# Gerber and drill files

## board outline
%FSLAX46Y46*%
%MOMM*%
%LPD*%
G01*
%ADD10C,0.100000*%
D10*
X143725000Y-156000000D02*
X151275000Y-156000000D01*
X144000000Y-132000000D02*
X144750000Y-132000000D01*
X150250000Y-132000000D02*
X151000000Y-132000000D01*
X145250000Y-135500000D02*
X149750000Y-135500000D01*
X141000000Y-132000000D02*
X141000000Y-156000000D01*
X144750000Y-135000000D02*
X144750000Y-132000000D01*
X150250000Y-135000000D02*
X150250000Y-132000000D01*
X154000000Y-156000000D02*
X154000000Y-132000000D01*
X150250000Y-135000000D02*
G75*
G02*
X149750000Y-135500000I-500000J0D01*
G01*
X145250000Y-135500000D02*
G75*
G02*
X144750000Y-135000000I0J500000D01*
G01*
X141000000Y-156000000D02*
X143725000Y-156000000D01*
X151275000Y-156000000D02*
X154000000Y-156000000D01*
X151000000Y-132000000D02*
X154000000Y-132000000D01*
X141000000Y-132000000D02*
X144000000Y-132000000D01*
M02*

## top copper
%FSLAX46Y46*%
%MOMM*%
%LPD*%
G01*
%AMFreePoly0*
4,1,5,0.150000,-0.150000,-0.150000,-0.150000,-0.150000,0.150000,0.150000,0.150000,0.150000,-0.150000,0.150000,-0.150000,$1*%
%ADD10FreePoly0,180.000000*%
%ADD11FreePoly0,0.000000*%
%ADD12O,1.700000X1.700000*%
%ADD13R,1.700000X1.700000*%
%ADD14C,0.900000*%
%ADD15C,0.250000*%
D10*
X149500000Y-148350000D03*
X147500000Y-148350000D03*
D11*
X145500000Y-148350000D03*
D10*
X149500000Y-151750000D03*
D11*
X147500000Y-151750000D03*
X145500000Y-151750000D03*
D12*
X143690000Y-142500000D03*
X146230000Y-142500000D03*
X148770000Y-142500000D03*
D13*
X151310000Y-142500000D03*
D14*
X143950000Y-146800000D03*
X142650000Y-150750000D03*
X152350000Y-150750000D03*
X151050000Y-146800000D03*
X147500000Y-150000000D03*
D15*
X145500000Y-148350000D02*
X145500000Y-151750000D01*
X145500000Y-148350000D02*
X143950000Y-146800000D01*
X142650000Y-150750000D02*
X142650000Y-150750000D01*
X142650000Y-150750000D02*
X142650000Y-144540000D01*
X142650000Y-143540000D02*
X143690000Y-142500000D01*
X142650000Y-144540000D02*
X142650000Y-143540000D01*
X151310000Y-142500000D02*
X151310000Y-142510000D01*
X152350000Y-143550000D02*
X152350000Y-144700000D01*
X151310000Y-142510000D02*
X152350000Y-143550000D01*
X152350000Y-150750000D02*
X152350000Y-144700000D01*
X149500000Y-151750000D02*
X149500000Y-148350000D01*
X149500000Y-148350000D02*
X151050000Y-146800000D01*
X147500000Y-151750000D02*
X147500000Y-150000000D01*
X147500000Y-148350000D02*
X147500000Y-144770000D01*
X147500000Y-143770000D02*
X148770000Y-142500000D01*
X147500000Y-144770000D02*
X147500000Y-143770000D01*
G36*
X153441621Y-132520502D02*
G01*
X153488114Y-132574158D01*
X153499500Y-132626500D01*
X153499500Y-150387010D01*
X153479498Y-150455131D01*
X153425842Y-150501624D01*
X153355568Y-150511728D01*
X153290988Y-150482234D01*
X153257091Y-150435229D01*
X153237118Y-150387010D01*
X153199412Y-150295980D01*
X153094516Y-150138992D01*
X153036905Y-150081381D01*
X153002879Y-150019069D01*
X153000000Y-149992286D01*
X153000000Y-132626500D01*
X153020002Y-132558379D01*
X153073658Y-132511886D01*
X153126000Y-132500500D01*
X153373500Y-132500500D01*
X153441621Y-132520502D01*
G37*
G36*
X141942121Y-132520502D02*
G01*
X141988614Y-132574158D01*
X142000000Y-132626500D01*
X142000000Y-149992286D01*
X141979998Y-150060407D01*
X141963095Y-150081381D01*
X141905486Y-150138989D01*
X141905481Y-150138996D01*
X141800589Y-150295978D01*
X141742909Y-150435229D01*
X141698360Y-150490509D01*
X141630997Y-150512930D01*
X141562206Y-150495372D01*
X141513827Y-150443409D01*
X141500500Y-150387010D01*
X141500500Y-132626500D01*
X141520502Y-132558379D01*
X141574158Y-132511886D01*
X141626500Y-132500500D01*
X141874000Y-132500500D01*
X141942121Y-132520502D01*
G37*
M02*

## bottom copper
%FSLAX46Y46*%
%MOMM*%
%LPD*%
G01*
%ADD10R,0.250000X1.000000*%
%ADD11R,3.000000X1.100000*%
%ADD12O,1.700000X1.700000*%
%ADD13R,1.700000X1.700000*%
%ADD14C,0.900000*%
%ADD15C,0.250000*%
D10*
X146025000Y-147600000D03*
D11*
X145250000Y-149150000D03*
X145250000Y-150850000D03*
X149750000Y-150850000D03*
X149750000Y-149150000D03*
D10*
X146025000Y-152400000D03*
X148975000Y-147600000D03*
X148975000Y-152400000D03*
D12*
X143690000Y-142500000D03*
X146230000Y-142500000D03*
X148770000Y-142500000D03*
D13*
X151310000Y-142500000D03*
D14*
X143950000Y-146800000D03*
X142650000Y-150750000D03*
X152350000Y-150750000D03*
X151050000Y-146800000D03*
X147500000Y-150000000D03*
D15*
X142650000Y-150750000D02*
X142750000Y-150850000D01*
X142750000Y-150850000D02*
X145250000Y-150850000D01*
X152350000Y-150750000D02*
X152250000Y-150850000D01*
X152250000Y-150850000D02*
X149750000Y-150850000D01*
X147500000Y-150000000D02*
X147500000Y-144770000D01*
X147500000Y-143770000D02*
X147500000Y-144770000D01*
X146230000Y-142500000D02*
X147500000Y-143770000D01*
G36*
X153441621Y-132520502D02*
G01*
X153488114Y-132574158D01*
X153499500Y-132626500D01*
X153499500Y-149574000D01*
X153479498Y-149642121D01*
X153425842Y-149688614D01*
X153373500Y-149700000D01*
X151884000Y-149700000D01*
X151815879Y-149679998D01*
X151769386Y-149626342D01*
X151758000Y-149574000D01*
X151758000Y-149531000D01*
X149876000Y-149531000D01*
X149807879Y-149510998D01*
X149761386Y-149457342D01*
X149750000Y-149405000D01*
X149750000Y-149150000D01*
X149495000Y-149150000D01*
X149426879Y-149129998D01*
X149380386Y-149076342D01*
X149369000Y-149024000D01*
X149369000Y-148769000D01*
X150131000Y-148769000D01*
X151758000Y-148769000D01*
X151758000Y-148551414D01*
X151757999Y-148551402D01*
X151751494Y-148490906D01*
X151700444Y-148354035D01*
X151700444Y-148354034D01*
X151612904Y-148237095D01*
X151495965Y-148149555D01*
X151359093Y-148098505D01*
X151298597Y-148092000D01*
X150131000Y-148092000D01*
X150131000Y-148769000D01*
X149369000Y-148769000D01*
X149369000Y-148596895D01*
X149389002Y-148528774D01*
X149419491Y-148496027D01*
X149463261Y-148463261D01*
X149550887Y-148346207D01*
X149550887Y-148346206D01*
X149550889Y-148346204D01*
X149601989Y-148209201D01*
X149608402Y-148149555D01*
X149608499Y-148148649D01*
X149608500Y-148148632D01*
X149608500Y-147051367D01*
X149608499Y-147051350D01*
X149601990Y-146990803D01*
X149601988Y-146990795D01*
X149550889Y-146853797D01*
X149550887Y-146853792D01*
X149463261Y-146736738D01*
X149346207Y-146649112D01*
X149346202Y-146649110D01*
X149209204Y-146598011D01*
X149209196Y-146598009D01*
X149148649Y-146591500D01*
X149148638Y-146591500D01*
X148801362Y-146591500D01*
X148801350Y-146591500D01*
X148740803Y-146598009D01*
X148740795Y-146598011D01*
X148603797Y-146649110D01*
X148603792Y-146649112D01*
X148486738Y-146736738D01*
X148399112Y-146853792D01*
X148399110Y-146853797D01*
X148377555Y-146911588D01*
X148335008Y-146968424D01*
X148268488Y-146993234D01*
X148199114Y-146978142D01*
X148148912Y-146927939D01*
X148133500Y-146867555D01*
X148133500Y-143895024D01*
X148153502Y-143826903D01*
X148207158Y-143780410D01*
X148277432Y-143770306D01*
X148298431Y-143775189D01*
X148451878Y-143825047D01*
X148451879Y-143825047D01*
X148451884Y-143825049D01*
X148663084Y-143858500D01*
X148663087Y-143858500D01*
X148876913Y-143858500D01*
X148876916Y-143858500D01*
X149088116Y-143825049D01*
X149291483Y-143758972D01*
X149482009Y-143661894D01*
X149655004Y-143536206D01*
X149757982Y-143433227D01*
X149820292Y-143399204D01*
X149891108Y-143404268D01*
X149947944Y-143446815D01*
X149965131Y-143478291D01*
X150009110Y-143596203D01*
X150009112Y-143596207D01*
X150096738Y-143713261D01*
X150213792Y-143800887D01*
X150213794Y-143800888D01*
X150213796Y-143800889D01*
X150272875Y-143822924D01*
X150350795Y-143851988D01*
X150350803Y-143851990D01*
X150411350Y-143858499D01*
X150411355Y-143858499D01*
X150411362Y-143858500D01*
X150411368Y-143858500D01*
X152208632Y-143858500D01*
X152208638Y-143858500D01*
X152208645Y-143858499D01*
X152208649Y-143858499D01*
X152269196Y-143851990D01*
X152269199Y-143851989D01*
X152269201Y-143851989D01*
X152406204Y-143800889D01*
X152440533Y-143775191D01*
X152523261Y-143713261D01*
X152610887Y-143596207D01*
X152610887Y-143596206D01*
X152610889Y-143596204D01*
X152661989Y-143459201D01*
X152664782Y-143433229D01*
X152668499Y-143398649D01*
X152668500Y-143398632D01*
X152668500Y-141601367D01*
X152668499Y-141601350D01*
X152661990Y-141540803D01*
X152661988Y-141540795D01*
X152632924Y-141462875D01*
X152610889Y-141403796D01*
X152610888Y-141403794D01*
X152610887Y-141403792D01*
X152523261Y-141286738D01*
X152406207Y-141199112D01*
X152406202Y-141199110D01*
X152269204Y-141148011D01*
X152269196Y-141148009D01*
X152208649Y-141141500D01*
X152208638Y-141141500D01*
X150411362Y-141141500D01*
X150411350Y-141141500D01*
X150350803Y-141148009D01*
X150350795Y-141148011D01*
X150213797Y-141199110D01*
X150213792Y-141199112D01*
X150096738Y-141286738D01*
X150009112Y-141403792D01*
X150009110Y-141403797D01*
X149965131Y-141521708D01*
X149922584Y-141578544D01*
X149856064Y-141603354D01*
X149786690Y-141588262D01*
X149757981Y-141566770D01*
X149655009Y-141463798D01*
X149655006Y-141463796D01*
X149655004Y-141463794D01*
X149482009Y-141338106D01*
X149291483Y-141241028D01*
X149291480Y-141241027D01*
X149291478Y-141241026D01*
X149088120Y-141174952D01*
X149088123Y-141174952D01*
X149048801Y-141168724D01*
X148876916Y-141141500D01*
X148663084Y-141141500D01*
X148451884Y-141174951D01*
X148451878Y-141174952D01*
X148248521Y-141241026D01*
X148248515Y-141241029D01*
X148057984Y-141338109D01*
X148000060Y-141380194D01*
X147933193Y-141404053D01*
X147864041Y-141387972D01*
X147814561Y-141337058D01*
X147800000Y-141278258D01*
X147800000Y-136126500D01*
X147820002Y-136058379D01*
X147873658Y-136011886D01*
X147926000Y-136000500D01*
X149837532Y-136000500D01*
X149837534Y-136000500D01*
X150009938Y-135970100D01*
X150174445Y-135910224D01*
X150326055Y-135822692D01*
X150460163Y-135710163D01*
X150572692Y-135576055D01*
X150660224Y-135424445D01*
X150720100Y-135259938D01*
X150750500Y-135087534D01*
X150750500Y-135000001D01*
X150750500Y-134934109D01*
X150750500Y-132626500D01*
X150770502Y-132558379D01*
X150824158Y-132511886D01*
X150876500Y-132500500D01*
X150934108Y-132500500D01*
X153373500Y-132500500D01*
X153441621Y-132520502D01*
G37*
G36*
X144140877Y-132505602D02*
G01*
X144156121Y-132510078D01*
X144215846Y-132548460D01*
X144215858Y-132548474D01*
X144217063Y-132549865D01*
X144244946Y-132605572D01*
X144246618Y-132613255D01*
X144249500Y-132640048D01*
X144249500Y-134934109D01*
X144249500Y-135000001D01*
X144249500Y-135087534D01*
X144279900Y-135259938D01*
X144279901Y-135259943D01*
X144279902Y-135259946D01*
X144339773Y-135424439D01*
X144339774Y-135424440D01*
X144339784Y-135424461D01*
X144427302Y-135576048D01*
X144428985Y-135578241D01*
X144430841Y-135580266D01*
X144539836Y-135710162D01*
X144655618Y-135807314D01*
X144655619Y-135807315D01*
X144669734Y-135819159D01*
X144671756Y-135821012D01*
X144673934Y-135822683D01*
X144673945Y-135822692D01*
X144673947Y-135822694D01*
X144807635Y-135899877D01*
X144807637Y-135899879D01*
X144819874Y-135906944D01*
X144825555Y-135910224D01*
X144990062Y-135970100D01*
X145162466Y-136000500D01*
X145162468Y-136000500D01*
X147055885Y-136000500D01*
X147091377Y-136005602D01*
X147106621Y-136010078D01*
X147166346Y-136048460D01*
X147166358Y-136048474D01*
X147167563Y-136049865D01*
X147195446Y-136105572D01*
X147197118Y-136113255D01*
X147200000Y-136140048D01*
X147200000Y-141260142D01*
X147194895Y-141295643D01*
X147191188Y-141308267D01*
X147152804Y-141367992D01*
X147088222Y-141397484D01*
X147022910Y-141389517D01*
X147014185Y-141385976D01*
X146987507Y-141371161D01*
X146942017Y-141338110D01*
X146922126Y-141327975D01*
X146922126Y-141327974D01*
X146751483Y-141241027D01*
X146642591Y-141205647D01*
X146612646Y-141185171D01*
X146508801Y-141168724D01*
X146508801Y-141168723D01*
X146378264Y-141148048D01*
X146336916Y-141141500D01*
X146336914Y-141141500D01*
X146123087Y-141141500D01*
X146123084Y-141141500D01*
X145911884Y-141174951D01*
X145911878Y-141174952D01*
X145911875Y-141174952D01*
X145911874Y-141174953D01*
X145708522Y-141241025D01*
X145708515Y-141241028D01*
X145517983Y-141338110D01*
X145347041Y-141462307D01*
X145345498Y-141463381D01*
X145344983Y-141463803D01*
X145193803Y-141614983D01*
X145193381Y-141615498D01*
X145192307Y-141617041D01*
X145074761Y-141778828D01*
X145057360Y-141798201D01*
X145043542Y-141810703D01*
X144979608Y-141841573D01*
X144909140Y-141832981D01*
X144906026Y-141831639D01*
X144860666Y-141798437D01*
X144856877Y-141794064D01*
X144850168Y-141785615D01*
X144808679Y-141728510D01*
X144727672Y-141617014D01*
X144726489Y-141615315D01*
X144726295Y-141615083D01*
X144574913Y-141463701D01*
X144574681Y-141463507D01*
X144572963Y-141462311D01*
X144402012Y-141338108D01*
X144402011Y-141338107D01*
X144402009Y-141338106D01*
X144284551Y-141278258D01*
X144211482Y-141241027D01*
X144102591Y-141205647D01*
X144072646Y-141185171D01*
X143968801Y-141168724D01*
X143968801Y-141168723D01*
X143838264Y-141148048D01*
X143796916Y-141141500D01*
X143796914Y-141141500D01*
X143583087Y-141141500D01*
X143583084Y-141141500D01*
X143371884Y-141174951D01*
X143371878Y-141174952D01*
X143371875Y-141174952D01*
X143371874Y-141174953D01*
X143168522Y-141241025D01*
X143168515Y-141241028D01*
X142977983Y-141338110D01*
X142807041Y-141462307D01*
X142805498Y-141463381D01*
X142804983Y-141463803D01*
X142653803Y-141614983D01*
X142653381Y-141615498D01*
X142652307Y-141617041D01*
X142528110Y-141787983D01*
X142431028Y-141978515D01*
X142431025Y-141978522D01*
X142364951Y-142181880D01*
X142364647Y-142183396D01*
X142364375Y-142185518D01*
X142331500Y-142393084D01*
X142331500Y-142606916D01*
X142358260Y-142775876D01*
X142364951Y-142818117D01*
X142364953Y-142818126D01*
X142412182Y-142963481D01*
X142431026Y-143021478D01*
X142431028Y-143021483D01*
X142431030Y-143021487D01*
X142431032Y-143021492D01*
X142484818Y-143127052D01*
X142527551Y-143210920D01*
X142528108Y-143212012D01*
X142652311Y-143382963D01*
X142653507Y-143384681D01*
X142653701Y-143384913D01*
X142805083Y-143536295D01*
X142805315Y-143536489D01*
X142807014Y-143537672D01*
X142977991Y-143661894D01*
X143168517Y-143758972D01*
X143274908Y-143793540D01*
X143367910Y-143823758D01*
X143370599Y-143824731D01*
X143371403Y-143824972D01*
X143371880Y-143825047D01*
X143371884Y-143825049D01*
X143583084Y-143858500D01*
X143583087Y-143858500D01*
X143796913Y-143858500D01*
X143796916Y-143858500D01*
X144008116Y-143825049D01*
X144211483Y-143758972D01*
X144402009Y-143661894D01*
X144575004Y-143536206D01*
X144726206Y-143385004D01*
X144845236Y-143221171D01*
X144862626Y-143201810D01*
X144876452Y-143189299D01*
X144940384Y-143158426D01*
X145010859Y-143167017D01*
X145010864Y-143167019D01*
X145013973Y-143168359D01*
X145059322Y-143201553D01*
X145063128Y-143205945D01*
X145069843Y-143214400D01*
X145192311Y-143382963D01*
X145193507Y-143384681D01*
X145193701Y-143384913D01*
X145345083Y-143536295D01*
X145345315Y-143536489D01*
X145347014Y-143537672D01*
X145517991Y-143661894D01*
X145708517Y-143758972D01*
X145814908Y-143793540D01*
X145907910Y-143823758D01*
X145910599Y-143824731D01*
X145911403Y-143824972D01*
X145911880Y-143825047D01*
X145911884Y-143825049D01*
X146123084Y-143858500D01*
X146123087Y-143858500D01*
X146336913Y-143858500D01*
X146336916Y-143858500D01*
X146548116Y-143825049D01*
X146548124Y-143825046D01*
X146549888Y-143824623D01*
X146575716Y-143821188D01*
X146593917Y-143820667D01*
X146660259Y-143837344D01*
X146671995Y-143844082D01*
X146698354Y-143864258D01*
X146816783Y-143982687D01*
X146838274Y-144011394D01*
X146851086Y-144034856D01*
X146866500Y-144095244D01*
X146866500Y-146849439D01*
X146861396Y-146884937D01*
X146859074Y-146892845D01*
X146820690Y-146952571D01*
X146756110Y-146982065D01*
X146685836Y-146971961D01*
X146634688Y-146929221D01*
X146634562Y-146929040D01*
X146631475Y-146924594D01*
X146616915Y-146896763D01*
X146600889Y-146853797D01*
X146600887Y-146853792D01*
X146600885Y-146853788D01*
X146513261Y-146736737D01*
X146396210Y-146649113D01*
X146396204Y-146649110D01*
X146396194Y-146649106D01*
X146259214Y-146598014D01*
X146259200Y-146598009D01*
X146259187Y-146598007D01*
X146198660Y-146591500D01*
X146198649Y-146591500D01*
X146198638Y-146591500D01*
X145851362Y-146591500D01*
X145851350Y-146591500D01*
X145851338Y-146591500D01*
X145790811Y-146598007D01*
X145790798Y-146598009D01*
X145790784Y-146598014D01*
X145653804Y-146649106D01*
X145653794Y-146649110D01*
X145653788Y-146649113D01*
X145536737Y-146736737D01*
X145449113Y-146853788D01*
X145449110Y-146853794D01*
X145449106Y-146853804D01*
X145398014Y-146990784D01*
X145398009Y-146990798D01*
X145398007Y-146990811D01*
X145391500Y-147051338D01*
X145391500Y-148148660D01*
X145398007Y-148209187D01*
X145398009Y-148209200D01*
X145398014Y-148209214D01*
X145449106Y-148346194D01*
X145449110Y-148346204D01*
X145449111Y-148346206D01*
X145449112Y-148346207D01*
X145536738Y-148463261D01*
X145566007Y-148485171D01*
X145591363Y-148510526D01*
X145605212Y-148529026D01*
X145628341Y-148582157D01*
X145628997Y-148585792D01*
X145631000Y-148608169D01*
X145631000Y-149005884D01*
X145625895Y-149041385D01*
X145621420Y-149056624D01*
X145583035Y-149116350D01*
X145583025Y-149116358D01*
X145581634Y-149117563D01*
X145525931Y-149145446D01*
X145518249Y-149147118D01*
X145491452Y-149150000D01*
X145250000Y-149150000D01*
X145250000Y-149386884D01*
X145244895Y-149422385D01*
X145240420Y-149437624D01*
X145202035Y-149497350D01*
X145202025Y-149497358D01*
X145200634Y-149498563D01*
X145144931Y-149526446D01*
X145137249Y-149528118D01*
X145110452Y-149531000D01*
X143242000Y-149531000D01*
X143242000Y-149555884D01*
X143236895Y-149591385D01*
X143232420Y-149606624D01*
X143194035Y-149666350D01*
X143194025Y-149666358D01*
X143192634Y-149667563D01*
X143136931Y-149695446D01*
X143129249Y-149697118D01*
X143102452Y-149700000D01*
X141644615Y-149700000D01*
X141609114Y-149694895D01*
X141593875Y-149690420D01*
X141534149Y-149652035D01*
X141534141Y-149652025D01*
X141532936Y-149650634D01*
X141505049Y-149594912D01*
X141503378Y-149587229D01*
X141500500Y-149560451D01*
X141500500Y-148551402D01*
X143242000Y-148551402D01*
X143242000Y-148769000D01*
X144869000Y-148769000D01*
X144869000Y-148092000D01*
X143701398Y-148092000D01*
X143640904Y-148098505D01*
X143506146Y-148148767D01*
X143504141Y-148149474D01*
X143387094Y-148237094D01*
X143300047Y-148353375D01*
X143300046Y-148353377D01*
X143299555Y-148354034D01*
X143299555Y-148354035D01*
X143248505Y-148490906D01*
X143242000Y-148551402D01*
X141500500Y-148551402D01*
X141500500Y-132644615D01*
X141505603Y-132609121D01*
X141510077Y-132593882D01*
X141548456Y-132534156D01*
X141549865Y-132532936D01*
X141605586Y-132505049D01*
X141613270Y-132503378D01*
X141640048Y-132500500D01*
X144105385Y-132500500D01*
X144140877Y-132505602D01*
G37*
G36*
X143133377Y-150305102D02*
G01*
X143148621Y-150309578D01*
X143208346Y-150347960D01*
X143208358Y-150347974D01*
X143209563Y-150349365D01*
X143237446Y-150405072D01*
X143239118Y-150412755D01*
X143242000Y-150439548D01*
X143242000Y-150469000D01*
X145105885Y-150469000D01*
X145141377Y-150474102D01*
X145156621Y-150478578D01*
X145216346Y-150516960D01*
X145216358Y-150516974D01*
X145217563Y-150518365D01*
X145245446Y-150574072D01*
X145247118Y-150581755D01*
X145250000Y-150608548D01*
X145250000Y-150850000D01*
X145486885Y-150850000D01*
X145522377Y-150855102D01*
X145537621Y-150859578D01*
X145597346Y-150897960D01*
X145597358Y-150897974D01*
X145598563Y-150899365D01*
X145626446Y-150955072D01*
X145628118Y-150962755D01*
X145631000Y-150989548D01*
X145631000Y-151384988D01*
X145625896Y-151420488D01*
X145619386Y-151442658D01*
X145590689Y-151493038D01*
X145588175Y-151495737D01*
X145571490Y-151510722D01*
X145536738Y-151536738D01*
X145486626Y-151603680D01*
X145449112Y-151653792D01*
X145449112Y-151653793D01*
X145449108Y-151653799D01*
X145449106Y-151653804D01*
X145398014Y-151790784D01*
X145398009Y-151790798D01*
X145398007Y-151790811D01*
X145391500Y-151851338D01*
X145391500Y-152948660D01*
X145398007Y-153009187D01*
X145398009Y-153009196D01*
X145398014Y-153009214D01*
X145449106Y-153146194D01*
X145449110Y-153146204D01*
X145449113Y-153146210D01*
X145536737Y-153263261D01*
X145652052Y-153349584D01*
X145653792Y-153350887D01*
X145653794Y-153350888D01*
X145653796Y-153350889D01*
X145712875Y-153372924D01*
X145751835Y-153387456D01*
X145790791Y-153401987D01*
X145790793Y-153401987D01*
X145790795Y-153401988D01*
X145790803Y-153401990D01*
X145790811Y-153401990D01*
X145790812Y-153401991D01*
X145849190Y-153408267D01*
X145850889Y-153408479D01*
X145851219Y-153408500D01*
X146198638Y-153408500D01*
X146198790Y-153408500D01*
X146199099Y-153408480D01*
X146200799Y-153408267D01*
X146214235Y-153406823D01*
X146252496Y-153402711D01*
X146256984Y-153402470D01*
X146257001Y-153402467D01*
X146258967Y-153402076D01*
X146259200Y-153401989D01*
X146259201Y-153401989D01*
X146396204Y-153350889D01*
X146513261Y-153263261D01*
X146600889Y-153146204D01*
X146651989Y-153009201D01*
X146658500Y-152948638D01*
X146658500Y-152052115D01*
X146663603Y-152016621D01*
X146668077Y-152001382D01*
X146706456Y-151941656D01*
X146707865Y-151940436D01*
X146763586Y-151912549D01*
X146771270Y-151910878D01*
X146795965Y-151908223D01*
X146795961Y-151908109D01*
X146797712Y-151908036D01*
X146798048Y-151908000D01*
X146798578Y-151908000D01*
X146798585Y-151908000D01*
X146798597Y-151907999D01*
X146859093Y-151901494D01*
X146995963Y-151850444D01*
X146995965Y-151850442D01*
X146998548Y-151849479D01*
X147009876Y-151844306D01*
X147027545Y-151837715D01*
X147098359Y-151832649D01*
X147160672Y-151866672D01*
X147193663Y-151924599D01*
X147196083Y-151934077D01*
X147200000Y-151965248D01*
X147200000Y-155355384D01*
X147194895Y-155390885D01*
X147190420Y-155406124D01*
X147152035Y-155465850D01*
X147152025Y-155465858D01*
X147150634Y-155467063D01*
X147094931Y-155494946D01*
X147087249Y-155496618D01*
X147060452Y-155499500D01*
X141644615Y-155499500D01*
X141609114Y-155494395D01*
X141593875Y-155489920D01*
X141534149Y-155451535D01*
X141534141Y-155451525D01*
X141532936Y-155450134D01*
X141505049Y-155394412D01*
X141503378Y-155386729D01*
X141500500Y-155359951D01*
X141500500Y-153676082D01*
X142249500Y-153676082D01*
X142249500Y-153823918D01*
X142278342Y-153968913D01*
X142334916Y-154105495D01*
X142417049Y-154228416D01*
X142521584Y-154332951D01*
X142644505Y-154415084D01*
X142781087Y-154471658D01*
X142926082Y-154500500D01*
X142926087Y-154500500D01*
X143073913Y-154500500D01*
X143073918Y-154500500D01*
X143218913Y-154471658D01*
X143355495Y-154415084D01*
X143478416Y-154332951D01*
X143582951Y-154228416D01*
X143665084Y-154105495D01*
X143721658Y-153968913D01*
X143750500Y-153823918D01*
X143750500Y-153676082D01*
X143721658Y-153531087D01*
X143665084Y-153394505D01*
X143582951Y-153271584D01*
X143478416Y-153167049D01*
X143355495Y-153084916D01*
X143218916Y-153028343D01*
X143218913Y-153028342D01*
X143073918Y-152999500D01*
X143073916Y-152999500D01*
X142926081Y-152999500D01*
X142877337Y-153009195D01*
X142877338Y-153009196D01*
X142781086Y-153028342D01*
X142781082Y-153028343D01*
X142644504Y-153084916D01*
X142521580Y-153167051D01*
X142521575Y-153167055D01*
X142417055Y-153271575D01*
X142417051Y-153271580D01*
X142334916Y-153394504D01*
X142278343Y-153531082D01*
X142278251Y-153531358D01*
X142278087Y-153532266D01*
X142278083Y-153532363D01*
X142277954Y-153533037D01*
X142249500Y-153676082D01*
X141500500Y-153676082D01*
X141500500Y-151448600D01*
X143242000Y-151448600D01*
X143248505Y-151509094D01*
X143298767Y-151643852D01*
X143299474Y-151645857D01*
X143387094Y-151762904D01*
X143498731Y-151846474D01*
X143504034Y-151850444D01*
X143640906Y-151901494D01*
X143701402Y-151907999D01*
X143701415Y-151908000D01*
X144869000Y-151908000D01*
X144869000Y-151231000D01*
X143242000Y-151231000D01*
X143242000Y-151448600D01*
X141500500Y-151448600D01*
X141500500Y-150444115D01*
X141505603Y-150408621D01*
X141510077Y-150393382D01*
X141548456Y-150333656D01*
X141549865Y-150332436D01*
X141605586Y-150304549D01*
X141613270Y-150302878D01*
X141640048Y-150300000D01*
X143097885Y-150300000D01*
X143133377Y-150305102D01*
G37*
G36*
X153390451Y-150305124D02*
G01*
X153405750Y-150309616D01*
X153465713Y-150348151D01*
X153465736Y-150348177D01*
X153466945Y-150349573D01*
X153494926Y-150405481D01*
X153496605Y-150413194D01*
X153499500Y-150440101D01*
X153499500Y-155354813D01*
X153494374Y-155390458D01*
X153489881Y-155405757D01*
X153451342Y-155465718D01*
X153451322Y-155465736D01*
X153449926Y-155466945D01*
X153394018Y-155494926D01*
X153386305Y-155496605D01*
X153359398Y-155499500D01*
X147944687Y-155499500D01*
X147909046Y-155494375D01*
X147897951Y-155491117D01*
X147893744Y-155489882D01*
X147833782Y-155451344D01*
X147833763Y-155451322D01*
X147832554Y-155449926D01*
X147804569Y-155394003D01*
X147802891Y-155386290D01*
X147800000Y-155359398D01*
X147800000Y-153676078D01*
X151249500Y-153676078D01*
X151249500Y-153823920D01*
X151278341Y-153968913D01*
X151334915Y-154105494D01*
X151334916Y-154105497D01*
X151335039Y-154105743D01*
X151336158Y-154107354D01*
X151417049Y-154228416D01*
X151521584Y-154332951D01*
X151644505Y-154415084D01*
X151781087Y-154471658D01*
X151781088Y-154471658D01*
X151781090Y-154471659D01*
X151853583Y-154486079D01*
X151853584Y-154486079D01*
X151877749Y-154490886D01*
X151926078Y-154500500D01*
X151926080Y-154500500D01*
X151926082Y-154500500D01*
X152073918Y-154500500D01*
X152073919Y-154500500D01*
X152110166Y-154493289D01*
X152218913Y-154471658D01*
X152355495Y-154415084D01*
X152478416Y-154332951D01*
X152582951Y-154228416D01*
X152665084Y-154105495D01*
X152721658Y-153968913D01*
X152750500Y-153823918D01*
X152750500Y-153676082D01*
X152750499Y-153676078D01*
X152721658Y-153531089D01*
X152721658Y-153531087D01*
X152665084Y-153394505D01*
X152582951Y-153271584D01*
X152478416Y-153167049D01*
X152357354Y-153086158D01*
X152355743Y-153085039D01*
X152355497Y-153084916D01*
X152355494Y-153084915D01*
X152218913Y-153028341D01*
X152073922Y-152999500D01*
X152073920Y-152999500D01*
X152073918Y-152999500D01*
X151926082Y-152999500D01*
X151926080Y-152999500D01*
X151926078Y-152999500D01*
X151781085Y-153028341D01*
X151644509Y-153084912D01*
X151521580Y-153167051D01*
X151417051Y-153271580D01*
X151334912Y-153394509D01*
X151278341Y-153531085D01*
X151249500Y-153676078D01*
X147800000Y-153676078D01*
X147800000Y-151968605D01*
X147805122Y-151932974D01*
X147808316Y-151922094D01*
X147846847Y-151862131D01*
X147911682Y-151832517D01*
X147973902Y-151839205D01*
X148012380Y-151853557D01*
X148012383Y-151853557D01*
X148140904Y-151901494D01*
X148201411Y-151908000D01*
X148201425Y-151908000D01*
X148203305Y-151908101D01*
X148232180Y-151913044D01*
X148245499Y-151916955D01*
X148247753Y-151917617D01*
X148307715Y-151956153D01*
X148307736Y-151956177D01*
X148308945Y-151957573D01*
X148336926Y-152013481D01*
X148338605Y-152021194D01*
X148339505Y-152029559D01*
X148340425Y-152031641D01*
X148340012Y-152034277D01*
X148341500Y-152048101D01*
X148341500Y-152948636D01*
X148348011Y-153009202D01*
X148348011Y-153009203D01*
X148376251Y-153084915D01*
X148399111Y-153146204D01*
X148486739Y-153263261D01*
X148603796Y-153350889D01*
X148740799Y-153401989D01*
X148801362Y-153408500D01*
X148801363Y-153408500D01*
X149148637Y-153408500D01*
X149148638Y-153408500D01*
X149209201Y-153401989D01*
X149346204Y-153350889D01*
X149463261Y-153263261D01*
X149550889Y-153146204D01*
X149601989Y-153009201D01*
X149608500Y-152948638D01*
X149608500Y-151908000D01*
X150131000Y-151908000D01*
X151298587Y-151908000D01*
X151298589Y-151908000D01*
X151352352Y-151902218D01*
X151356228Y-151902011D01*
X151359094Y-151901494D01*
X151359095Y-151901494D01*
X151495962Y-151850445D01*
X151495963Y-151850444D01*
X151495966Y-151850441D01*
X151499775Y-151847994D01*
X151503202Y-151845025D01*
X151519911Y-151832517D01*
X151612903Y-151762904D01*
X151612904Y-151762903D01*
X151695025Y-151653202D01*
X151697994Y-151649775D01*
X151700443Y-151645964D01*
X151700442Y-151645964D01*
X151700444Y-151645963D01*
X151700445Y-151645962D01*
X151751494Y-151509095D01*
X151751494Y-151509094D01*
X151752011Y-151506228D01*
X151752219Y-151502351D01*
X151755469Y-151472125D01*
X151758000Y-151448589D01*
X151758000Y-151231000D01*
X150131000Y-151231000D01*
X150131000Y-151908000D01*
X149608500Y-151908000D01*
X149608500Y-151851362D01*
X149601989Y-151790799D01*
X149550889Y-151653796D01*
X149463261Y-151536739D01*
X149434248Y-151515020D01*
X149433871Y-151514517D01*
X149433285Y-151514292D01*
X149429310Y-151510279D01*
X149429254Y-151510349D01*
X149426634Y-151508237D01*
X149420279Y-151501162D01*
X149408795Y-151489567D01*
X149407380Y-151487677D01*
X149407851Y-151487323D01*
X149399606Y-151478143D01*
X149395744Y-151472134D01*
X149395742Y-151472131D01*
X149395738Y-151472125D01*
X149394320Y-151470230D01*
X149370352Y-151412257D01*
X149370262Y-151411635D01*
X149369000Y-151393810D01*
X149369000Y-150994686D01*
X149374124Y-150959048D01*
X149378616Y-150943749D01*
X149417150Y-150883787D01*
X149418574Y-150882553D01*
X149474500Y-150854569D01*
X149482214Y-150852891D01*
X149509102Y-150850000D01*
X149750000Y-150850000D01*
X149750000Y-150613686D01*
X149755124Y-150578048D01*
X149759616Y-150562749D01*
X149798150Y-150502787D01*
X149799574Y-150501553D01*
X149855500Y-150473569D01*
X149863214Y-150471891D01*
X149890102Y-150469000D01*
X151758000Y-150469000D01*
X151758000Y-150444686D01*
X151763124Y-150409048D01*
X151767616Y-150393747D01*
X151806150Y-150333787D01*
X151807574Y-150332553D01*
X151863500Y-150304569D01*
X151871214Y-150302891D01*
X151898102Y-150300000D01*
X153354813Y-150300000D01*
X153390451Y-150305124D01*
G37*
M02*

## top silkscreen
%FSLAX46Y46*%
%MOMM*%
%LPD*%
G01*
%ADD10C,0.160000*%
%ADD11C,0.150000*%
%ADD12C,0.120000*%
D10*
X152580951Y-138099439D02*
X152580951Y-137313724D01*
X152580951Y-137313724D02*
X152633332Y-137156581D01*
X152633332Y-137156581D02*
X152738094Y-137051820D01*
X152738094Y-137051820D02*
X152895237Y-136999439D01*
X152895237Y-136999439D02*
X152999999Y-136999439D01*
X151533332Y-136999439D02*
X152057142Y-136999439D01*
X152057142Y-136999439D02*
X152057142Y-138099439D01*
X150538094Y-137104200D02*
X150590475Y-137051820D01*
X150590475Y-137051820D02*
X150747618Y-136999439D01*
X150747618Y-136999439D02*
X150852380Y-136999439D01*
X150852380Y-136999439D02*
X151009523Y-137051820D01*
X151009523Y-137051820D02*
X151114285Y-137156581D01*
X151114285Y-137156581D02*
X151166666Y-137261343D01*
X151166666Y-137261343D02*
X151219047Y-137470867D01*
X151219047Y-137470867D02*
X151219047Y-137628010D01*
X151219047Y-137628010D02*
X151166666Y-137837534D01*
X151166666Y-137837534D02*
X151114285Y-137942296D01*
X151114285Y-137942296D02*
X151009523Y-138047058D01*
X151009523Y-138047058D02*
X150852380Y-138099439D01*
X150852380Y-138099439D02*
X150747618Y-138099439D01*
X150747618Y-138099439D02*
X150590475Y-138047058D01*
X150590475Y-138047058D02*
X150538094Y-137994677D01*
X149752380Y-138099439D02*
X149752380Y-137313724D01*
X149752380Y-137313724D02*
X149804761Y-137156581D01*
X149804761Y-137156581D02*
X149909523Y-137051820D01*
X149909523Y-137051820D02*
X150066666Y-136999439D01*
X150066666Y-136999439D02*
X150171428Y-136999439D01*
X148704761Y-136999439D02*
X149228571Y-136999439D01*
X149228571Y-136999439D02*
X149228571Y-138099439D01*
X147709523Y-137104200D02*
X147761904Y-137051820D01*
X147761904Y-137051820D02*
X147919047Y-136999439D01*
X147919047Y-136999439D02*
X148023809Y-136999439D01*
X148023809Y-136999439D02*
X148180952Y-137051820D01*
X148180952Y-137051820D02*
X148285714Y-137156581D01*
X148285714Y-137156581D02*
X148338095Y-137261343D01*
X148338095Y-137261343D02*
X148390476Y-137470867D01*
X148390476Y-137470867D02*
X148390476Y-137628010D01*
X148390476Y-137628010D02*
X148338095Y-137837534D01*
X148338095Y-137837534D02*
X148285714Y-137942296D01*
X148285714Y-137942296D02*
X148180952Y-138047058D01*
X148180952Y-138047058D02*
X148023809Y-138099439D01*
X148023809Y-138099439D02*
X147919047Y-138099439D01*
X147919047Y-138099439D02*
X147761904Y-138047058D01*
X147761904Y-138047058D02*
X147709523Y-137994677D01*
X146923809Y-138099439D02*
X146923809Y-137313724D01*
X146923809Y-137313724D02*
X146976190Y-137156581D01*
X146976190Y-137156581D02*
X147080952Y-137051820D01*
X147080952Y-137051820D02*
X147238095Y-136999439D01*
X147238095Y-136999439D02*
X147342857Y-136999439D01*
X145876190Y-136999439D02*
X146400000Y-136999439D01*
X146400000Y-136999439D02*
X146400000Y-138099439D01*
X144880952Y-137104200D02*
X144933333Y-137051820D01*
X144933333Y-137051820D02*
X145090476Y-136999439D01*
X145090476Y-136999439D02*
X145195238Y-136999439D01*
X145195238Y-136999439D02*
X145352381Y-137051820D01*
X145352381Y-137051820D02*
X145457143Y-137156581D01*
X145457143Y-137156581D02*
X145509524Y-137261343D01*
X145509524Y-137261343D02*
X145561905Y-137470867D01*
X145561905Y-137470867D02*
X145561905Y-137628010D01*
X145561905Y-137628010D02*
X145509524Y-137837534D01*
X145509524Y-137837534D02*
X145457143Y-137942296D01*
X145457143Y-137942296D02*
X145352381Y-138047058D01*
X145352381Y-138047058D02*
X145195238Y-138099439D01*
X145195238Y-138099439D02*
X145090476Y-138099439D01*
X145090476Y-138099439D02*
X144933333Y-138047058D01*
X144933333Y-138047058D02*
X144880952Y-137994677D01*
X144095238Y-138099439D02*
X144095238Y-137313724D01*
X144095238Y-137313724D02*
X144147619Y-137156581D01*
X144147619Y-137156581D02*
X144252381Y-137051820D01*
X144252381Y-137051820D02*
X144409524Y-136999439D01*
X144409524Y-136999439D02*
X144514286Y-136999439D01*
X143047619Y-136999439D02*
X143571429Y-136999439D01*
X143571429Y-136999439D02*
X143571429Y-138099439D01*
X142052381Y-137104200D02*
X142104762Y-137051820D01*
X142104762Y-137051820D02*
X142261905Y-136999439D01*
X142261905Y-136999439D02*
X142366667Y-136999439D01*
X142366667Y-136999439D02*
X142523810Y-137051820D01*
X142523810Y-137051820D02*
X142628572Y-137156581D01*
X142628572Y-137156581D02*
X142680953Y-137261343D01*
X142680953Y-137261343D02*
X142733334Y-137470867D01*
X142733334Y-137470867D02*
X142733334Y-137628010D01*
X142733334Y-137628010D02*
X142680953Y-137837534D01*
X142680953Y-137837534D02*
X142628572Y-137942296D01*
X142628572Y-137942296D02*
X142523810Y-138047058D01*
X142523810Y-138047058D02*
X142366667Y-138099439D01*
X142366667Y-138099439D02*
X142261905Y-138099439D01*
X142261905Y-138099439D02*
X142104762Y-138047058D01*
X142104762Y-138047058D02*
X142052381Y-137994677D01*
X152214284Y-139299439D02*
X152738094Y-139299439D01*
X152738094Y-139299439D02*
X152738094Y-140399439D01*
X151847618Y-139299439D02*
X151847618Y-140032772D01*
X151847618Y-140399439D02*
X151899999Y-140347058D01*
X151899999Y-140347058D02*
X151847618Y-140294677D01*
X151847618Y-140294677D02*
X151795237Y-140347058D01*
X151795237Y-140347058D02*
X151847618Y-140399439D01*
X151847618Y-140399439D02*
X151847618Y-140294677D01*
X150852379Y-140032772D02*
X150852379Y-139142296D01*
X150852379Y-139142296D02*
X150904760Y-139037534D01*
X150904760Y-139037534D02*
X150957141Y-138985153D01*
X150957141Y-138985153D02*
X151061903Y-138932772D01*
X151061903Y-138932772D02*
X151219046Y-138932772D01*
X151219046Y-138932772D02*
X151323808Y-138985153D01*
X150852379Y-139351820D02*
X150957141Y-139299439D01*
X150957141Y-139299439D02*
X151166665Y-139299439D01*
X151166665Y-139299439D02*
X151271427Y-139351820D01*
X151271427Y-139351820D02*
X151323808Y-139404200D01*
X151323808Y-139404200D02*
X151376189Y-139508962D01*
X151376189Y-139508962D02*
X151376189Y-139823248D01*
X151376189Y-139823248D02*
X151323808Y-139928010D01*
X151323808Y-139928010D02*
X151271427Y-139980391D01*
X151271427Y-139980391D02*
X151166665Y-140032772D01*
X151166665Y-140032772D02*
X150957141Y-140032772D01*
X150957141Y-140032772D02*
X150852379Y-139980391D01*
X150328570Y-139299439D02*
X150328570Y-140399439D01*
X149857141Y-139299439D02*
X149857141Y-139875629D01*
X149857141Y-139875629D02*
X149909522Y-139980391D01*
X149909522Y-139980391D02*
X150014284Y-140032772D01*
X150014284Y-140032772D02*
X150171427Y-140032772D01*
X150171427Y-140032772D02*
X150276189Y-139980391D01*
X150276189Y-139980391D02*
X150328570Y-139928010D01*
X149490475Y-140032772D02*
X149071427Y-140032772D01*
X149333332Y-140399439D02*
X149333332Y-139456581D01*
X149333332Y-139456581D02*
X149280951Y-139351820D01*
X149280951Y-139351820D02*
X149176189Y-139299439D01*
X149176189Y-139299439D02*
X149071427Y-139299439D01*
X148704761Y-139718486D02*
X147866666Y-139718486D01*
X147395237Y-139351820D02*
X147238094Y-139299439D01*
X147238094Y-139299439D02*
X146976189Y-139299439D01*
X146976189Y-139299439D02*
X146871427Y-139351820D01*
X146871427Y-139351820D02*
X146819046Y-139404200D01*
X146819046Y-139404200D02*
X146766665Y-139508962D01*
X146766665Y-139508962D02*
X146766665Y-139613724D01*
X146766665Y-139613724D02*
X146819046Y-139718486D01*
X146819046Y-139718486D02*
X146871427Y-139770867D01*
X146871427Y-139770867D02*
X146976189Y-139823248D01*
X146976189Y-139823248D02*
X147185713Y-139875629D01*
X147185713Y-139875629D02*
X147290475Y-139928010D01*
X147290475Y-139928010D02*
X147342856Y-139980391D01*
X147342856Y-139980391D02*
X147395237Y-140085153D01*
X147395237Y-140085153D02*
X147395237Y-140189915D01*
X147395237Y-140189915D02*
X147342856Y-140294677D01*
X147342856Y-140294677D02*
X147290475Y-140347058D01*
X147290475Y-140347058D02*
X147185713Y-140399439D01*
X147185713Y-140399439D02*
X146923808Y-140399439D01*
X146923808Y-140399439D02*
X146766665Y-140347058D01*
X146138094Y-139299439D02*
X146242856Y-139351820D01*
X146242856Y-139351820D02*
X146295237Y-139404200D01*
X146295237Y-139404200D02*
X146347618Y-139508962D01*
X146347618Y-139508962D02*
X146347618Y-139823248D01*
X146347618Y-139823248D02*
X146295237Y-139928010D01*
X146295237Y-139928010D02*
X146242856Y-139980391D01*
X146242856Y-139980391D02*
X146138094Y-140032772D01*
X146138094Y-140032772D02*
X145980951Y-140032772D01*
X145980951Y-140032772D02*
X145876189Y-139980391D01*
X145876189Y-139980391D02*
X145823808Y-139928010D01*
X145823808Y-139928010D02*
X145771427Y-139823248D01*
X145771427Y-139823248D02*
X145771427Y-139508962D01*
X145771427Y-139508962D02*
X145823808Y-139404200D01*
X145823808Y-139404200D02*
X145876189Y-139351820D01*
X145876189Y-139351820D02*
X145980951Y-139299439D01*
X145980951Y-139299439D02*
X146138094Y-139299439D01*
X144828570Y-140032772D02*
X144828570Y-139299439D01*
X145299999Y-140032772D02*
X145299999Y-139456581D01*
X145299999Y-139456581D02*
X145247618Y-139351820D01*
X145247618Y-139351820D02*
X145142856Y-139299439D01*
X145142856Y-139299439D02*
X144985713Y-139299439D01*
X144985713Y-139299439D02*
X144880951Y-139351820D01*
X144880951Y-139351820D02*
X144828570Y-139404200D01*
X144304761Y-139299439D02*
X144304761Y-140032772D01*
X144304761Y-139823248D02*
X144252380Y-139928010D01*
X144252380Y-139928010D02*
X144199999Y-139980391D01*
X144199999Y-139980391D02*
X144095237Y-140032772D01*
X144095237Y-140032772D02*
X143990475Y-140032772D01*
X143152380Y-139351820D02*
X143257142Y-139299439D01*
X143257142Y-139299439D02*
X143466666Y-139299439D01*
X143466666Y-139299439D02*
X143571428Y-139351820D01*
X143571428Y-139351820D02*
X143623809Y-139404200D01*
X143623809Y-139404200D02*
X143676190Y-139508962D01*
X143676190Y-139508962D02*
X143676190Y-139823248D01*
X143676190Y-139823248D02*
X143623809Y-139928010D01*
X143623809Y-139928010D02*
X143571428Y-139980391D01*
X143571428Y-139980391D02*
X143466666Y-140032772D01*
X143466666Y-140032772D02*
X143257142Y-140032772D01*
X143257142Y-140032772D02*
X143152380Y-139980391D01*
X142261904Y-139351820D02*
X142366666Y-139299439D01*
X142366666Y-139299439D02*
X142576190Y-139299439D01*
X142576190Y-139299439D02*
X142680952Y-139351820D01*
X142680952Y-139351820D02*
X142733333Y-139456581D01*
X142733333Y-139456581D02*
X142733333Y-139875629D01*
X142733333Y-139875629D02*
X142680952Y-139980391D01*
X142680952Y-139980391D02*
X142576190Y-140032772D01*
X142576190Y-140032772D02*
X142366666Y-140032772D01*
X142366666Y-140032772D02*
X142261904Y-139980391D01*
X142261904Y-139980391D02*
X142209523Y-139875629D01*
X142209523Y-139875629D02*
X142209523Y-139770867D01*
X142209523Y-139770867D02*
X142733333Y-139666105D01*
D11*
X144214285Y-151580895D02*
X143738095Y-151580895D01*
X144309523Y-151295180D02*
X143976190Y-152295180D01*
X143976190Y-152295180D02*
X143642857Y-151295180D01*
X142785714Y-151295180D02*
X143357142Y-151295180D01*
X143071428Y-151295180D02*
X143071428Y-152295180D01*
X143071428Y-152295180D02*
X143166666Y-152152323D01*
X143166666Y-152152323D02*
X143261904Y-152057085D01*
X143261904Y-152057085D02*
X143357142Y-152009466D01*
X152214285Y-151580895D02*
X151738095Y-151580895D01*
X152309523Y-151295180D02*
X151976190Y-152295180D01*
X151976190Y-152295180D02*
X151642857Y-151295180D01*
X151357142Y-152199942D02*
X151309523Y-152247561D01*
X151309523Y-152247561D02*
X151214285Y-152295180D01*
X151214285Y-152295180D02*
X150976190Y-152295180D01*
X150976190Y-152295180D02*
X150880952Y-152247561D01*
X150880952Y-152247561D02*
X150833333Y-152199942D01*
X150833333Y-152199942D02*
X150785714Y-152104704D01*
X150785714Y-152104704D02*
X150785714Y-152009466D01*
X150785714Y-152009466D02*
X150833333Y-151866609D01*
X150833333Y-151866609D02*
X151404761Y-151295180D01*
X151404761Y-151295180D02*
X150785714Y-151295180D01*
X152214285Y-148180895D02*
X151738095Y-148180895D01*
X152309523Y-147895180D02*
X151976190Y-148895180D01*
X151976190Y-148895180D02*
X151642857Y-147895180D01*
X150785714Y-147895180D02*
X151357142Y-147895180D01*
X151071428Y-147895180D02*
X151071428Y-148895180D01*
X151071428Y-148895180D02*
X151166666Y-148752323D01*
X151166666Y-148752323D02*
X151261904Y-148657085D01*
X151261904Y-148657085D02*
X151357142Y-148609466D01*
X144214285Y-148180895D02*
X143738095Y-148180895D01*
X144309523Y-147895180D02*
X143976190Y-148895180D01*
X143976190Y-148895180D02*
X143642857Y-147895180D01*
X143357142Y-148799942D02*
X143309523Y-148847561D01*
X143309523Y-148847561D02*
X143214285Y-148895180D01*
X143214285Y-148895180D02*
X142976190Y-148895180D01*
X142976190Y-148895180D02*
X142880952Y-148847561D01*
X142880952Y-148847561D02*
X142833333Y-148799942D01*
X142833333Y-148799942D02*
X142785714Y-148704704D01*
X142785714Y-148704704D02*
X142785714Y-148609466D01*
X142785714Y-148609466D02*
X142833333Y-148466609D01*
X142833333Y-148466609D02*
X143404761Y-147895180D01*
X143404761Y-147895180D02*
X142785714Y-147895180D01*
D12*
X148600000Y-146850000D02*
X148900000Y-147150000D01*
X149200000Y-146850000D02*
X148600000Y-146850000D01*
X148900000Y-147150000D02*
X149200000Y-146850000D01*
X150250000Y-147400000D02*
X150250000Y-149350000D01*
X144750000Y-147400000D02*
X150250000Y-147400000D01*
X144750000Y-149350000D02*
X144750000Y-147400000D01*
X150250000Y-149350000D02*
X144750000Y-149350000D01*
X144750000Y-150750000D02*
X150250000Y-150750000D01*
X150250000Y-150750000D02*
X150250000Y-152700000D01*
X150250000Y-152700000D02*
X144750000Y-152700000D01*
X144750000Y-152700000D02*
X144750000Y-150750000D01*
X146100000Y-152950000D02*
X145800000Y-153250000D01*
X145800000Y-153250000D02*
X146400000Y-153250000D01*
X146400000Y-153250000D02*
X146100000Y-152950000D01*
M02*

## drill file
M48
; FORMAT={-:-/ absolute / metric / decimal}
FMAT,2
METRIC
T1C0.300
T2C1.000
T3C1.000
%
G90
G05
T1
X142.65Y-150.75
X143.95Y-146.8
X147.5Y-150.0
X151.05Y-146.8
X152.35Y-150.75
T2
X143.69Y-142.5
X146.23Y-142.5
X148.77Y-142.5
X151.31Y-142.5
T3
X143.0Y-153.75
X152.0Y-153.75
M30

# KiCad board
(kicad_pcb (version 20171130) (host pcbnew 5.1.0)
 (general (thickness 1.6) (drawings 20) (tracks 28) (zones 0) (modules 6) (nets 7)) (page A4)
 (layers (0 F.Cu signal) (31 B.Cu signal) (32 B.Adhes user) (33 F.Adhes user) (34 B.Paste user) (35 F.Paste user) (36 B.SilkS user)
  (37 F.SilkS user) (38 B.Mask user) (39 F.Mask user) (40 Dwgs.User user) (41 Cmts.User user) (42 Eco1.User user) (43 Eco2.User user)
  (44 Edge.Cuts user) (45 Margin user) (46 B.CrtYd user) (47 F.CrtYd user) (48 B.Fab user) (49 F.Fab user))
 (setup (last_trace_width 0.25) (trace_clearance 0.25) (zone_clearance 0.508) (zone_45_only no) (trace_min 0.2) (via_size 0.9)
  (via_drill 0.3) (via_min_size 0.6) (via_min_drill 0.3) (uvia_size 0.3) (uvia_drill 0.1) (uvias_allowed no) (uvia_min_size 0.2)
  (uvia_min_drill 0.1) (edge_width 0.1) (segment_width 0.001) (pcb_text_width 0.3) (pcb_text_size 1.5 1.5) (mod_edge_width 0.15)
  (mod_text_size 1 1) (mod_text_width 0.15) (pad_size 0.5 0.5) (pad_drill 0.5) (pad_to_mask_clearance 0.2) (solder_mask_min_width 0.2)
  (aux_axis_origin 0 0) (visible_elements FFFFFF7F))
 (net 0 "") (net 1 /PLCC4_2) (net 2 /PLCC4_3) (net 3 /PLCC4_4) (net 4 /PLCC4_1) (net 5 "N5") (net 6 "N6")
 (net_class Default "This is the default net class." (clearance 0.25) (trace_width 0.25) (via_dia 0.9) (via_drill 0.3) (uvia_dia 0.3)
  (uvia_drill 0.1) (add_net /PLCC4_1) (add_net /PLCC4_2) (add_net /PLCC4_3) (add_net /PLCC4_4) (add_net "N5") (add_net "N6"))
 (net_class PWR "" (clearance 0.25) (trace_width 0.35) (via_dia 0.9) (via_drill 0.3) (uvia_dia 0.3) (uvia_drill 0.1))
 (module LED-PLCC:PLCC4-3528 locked (layer B.Cu) (at 147.5 150 270)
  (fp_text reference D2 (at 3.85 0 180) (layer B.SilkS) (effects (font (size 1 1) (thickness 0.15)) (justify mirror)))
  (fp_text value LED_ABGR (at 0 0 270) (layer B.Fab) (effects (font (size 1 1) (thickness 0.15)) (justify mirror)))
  (pad ~ smd rect (at -2.4 1.475 270) (size 1 0.25) (layers B.Cu B.Paste B.Mask))
  (pad 2 smd rect (at -0.85 2.25 270) (size 1.1 3) (layers B.Cu B.Paste B.Mask) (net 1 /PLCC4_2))
  (pad 3 smd rect (at 0.85 2.25 270) (size 1.1 3) (layers B.Cu B.Paste B.Mask) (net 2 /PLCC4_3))
  (pad 4 smd rect (at 0.85 -2.25 270) (size 1.1 3) (layers B.Cu B.Paste B.Mask) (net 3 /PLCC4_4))
  (pad 1 smd rect (at -0.85 -2.25 270) (size 1.1 3) (layers B.Cu B.Paste B.Mask) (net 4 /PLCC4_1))
  (pad ~ smd rect (at 2.4 1.475 270) (size 1 0.25) (layers B.Cu B.Paste B.Mask))
  (pad ~ smd rect (at -2.4 -1.475 270) (size 1 0.25) (layers B.Cu B.Paste B.Mask))
  (pad ~ smd rect (at 2.4 -1.475 270) (size 1 0.25) (layers B.Cu B.Paste B.Mask)))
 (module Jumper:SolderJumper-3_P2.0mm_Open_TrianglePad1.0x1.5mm (layer F.Cu) (at 147.5 148.35 180)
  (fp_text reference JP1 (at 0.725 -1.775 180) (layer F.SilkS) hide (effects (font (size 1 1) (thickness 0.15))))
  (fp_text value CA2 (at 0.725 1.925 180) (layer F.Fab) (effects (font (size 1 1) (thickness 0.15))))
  (fp_line (start -1.1 1.5) (end -1.4 1.2) (layer F.SilkS) (width 0.12))
  (fp_line (start -1.7 1.5) (end -1.1 1.5) (layer F.SilkS) (width 0.12))
  (fp_line (start -1.4 1.2) (end -1.7 1.5) (layer F.SilkS) (width 0.12))
  (fp_line (start -2.75 0.95) (end -2.75 -1) (layer F.SilkS) (width 0.12))
  (fp_line (start 2.75 0.95) (end -2.75 0.95) (layer F.SilkS) (width 0.12))
  (fp_line (start 2.75 -1) (end 2.75 0.95) (layer F.SilkS) (width 0.12))
  (fp_line (start -2.75 -1) (end 2.75 -1) (layer F.SilkS) (width 0.12))
  (pad "" smd rect (at 1.2 0 180) (size 1.5 1.5) (layers F.Mask))
  (pad "" smd rect (at -1.2 0 180) (size 1.5 1.5) (layers F.Mask))
  (pad 1 smd custom (at -2 0 180) (size 0.3 0.3) (layers F.Cu F.Mask) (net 4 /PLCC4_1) (zone_connect 0)
   (options (clearance outline) (anchor rect)) (primitives))
  (pad 2 smd custom (at 0 0 180) (size 0.3 0.3) (layers F.Cu) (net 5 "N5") (zone_connect 0) (options (clearance outline) (anchor rect))
   (primitives))
  (pad 3 smd custom (at 2 0) (size 0.3 0.3) (layers F.Cu F.Mask) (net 1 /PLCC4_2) (zone_connect 0)
   (options (clearance outline) (anchor rect)) (primitives)))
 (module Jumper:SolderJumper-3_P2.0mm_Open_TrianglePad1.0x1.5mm (layer F.Cu) (at 147.5 151.75)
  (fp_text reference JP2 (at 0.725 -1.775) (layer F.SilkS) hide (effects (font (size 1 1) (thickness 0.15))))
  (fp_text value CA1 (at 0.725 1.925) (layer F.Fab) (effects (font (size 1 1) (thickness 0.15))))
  (fp_line (start -2.75 -1) (end 2.75 -1) (layer F.SilkS) (width 0.12))
  (fp_line (start 2.75 -1) (end 2.75 0.95) (layer F.SilkS) (width 0.12))
  (fp_line (start 2.75 0.95) (end -2.75 0.95) (layer F.SilkS) (width 0.12))
  (fp_line (start -2.75 0.95) (end -2.75 -1) (layer F.SilkS) (width 0.12))
  (fp_line (start -1.4 1.2) (end -1.7 1.5) (layer F.SilkS) (width 0.12))
  (fp_line (start -1.7 1.5) (end -1.1 1.5) (layer F.SilkS) (width 0.12))
  (fp_line (start -1.1 1.5) (end -1.4 1.2) (layer F.SilkS) (width 0.12))
  (pad 3 smd custom (at 2 0 180) (size 0.3 0.3) (layers F.Cu F.Mask) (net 4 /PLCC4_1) (zone_connect 0)
   (options (clearance outline) (anchor rect)) (primitives))
  (pad 2 smd custom (at 0 0) (size 0.3 0.3) (layers F.Cu) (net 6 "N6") (zone_connect 0) (options (clearance outline) (anchor rect))
   (primitives))
  (pad 1 smd custom (at -2 0) (size 0.3 0.3) (layers F.Cu F.Mask) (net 1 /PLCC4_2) (zone_connect 0)
   (options (clearance outline) (anchor rect)) (primitives))
  (pad "" smd rect (at -1.2 0) (size 1.5 1.5) (layers F.Mask)) (pad "" smd rect (at 1.2 0) (size 1.5 1.5) (layers F.Mask)))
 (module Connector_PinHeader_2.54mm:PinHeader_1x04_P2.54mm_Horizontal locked (layer B.Cu) (at 151.31 142.5 90)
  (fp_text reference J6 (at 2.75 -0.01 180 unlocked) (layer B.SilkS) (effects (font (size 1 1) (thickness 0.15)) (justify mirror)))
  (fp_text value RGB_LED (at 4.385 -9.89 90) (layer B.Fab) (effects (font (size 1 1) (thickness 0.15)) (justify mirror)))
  (pad 4 thru_hole oval (at 0 -7.62 90) (size 1.7 1.7) (drill 1) (layers *.Cu *.Mask) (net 2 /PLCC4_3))
  (pad 3 thru_hole oval (at 0 -5.08 90) (size 1.7 1.7) (drill 1) (layers *.Cu *.Mask) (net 6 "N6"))
  (pad 2 thru_hole oval (at 0 -2.54 90) (size 1.7 1.7) (drill 1) (layers *.Cu *.Mask) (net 5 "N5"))
  (pad 1 thru_hole rect (at 0 0 90) (size 1.7 1.7) (drill 1) (layers *.Cu *.Mask) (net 3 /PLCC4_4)))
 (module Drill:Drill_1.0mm (layer F.Cu) (at 143 153.75)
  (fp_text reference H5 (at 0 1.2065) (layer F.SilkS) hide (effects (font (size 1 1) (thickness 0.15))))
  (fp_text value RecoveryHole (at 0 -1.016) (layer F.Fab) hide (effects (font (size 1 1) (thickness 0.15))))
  (pad "" np_thru_hole circle (at 0 0) (size 1 1) (drill 1) (layers *.Cu *.Mask) (solder_mask_margin 0.0001) (clearance 0.25)))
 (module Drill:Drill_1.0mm (layer F.Cu) (at 152 153.75)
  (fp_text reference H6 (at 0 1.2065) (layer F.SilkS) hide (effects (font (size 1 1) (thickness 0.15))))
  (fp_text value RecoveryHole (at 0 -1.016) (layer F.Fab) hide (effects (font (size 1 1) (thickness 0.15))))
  (pad "" np_thru_hole circle (at 0 0) (size 1 1) (drill 1) (layers *.Cu *.Mask) (solder_mask_margin 0.0001) (clearance 0.25)))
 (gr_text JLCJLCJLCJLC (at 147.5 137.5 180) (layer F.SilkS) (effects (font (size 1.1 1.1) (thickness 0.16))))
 (gr_line (start 143.725 156) (end 151.275 156) (layer Edge.Cuts) (width 0.1))
 (gr_line (start 144 132) (end 144.75 132) (layer Edge.Cuts) (width 0.1))
 (gr_line (start 150.25 132) (end 151 132) (layer Edge.Cuts) (width 0.1))
 (gr_line (start 145.25 135.5) (end 149.75 135.5) (layer Edge.Cuts) (width 0.1))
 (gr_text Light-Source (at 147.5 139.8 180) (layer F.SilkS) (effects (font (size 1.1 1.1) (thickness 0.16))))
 (gr_line (start 141 132) (end 141 156) (layer Edge.Cuts) (width 0.1))
 (gr_line (start 144.75 135) (end 144.75 132) (layer Edge.Cuts) (width 0.1))
 (gr_line (start 150.25 135) (end 150.25 132) (layer Edge.Cuts) (width 0.1))
 (gr_line (start 154 156) (end 154 132) (layer Edge.Cuts) (width 0.1))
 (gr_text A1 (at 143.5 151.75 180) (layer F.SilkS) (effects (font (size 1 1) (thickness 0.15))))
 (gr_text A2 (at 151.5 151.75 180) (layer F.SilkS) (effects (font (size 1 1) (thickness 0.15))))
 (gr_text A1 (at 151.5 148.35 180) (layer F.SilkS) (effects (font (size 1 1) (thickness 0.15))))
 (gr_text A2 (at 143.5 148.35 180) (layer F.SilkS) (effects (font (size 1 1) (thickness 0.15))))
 (gr_arc (start 149.75 135) (end 149.75 135.5) (angle -90) (layer Edge.Cuts) (width 0.1))
 (gr_arc (start 145.25 135) (end 144.75 135) (angle -90) (layer Edge.Cuts) (width 0.1))
 (gr_line (start 141 156) (end 143.725 156) (layer Edge.Cuts) (width 0.1))
 (gr_line (start 151.275 156) (end 154 156) (layer Edge.Cuts) (width 0.1))
 (gr_line (start 151 132) (end 154 132) (angle 90) (layer Edge.Cuts) (width 0.1))
 (gr_line (start 141 132) (end 144 132) (angle 90) (layer Edge.Cuts) (width 0.1))
 (segment (start 145.5 148.35) (end 145.5 151.75) (width 0.25) (layer F.Cu) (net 1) (status C00000))
 (via (at 143.95 146.8) (size 0.9) (drill 0.3) (layers F.Cu B.Cu) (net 1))
 (segment (start 145.5 148.35) (end 143.95 146.8) (width 0.25) (layer F.Cu) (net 1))
 (segment (start 142.65 150.75) (end 142.65 150.75) (width 0.25) (layer F.Cu) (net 2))
 (via (at 142.65 150.75) (size 0.9) (drill 0.3) (layers F.Cu B.Cu) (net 2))
 (segment (start 142.65 150.75) (end 142.75 150.85) (width 0.25) (layer B.Cu) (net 2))
 (segment (start 142.75 150.85) (end 145.25 150.85) (width 0.25) (layer B.Cu) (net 2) (status 800000))
 (segment (start 142.65 150.75) (end 142.65 144.54) (width 0.25) (layer F.Cu) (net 2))
 (segment (start 142.65 143.54) (end 143.69 142.5) (width 0.25) (layer F.Cu) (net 2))
 (segment (start 142.65 144.54) (end 142.65 143.54) (width 0.25) (layer F.Cu) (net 2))
 (via (at 152.35 150.75) (size 0.9) (drill 0.3) (layers F.Cu B.Cu) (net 3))
 (segment (start 152.35 150.75) (end 152.25 150.85) (width 0.25) (layer B.Cu) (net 3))
 (segment (start 152.25 150.85) (end 149.75 150.85) (width 0.25) (layer B.Cu) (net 3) (status 800000))
 (segment (start 151.31 142.5) (end 151.31 142.51) (width 0.25) (layer F.Cu) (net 3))
 (segment (start 152.35 143.55) (end 152.35 144.7) (width 0.25) (layer F.Cu) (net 3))
 (segment (start 151.31 142.51) (end 152.35 143.55) (width 0.25) (layer F.Cu) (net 3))
 (segment (start 152.35 150.75) (end 152.35 144.7) (width 0.25) (layer F.Cu) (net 3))
 (segment (start 149.5 151.75) (end 149.5 148.35) (width 0.25) (layer F.Cu) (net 4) (status C00000))
 (via (at 151.05 146.8) (size 0.9) (drill 0.3) (layers F.Cu B.Cu) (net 4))
 (segment (start 149.5 148.35) (end 151.05 146.8) (width 0.25) (layer F.Cu) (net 4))
 (segment (start 147.5 151.75) (end 147.5 150) (width 0.25) (layer F.Cu) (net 6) (status 400000))
 (via (at 147.5 150) (size 0.9) (drill 0.3) (layers F.Cu B.Cu) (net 6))
 (segment (start 147.5 150) (end 147.5 144.77) (width 0.25) (layer B.Cu) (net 6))
 (segment (start 147.5 143.77) (end 147.5 144.77) (width 0.25) (layer B.Cu) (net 6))
 (segment (start 146.23 142.5) (end 147.5 143.77) (width 0.25) (layer B.Cu) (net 6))
 (segment (start 147.5 148.35) (end 147.5 144.77) (width 0.25) (layer F.Cu) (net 5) (status 400000))
 (segment (start 147.5 143.77) (end 148.77 142.5) (width 0.25) (layer F.Cu) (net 5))
 (segment (start 147.5 144.77) (end 147.5 143.77) (width 0.25) (layer F.Cu) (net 5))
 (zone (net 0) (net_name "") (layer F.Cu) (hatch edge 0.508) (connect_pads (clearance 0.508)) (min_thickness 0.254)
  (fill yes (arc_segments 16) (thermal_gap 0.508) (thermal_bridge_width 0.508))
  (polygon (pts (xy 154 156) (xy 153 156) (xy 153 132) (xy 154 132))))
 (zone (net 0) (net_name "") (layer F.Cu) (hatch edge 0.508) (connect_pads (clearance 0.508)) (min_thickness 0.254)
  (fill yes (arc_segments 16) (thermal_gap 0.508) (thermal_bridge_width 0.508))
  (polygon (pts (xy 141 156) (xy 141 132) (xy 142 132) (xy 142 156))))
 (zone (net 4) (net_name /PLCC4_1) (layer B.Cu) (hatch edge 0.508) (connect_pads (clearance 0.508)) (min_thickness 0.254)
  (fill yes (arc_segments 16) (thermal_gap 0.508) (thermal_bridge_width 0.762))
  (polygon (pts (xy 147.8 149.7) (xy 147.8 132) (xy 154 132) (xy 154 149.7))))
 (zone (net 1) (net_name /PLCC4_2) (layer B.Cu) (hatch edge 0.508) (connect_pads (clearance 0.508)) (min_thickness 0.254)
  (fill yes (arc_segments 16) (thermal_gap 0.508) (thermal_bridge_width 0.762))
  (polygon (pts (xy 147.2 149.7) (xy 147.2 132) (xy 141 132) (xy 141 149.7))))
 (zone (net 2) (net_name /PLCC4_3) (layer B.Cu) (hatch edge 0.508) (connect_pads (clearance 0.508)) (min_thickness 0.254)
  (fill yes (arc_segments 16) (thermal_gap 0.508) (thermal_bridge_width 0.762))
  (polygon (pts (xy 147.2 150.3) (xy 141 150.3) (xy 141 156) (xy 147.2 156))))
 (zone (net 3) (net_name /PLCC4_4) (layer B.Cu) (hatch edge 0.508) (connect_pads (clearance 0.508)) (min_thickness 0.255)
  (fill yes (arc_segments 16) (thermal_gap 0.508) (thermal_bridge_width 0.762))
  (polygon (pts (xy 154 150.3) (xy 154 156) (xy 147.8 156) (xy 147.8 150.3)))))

